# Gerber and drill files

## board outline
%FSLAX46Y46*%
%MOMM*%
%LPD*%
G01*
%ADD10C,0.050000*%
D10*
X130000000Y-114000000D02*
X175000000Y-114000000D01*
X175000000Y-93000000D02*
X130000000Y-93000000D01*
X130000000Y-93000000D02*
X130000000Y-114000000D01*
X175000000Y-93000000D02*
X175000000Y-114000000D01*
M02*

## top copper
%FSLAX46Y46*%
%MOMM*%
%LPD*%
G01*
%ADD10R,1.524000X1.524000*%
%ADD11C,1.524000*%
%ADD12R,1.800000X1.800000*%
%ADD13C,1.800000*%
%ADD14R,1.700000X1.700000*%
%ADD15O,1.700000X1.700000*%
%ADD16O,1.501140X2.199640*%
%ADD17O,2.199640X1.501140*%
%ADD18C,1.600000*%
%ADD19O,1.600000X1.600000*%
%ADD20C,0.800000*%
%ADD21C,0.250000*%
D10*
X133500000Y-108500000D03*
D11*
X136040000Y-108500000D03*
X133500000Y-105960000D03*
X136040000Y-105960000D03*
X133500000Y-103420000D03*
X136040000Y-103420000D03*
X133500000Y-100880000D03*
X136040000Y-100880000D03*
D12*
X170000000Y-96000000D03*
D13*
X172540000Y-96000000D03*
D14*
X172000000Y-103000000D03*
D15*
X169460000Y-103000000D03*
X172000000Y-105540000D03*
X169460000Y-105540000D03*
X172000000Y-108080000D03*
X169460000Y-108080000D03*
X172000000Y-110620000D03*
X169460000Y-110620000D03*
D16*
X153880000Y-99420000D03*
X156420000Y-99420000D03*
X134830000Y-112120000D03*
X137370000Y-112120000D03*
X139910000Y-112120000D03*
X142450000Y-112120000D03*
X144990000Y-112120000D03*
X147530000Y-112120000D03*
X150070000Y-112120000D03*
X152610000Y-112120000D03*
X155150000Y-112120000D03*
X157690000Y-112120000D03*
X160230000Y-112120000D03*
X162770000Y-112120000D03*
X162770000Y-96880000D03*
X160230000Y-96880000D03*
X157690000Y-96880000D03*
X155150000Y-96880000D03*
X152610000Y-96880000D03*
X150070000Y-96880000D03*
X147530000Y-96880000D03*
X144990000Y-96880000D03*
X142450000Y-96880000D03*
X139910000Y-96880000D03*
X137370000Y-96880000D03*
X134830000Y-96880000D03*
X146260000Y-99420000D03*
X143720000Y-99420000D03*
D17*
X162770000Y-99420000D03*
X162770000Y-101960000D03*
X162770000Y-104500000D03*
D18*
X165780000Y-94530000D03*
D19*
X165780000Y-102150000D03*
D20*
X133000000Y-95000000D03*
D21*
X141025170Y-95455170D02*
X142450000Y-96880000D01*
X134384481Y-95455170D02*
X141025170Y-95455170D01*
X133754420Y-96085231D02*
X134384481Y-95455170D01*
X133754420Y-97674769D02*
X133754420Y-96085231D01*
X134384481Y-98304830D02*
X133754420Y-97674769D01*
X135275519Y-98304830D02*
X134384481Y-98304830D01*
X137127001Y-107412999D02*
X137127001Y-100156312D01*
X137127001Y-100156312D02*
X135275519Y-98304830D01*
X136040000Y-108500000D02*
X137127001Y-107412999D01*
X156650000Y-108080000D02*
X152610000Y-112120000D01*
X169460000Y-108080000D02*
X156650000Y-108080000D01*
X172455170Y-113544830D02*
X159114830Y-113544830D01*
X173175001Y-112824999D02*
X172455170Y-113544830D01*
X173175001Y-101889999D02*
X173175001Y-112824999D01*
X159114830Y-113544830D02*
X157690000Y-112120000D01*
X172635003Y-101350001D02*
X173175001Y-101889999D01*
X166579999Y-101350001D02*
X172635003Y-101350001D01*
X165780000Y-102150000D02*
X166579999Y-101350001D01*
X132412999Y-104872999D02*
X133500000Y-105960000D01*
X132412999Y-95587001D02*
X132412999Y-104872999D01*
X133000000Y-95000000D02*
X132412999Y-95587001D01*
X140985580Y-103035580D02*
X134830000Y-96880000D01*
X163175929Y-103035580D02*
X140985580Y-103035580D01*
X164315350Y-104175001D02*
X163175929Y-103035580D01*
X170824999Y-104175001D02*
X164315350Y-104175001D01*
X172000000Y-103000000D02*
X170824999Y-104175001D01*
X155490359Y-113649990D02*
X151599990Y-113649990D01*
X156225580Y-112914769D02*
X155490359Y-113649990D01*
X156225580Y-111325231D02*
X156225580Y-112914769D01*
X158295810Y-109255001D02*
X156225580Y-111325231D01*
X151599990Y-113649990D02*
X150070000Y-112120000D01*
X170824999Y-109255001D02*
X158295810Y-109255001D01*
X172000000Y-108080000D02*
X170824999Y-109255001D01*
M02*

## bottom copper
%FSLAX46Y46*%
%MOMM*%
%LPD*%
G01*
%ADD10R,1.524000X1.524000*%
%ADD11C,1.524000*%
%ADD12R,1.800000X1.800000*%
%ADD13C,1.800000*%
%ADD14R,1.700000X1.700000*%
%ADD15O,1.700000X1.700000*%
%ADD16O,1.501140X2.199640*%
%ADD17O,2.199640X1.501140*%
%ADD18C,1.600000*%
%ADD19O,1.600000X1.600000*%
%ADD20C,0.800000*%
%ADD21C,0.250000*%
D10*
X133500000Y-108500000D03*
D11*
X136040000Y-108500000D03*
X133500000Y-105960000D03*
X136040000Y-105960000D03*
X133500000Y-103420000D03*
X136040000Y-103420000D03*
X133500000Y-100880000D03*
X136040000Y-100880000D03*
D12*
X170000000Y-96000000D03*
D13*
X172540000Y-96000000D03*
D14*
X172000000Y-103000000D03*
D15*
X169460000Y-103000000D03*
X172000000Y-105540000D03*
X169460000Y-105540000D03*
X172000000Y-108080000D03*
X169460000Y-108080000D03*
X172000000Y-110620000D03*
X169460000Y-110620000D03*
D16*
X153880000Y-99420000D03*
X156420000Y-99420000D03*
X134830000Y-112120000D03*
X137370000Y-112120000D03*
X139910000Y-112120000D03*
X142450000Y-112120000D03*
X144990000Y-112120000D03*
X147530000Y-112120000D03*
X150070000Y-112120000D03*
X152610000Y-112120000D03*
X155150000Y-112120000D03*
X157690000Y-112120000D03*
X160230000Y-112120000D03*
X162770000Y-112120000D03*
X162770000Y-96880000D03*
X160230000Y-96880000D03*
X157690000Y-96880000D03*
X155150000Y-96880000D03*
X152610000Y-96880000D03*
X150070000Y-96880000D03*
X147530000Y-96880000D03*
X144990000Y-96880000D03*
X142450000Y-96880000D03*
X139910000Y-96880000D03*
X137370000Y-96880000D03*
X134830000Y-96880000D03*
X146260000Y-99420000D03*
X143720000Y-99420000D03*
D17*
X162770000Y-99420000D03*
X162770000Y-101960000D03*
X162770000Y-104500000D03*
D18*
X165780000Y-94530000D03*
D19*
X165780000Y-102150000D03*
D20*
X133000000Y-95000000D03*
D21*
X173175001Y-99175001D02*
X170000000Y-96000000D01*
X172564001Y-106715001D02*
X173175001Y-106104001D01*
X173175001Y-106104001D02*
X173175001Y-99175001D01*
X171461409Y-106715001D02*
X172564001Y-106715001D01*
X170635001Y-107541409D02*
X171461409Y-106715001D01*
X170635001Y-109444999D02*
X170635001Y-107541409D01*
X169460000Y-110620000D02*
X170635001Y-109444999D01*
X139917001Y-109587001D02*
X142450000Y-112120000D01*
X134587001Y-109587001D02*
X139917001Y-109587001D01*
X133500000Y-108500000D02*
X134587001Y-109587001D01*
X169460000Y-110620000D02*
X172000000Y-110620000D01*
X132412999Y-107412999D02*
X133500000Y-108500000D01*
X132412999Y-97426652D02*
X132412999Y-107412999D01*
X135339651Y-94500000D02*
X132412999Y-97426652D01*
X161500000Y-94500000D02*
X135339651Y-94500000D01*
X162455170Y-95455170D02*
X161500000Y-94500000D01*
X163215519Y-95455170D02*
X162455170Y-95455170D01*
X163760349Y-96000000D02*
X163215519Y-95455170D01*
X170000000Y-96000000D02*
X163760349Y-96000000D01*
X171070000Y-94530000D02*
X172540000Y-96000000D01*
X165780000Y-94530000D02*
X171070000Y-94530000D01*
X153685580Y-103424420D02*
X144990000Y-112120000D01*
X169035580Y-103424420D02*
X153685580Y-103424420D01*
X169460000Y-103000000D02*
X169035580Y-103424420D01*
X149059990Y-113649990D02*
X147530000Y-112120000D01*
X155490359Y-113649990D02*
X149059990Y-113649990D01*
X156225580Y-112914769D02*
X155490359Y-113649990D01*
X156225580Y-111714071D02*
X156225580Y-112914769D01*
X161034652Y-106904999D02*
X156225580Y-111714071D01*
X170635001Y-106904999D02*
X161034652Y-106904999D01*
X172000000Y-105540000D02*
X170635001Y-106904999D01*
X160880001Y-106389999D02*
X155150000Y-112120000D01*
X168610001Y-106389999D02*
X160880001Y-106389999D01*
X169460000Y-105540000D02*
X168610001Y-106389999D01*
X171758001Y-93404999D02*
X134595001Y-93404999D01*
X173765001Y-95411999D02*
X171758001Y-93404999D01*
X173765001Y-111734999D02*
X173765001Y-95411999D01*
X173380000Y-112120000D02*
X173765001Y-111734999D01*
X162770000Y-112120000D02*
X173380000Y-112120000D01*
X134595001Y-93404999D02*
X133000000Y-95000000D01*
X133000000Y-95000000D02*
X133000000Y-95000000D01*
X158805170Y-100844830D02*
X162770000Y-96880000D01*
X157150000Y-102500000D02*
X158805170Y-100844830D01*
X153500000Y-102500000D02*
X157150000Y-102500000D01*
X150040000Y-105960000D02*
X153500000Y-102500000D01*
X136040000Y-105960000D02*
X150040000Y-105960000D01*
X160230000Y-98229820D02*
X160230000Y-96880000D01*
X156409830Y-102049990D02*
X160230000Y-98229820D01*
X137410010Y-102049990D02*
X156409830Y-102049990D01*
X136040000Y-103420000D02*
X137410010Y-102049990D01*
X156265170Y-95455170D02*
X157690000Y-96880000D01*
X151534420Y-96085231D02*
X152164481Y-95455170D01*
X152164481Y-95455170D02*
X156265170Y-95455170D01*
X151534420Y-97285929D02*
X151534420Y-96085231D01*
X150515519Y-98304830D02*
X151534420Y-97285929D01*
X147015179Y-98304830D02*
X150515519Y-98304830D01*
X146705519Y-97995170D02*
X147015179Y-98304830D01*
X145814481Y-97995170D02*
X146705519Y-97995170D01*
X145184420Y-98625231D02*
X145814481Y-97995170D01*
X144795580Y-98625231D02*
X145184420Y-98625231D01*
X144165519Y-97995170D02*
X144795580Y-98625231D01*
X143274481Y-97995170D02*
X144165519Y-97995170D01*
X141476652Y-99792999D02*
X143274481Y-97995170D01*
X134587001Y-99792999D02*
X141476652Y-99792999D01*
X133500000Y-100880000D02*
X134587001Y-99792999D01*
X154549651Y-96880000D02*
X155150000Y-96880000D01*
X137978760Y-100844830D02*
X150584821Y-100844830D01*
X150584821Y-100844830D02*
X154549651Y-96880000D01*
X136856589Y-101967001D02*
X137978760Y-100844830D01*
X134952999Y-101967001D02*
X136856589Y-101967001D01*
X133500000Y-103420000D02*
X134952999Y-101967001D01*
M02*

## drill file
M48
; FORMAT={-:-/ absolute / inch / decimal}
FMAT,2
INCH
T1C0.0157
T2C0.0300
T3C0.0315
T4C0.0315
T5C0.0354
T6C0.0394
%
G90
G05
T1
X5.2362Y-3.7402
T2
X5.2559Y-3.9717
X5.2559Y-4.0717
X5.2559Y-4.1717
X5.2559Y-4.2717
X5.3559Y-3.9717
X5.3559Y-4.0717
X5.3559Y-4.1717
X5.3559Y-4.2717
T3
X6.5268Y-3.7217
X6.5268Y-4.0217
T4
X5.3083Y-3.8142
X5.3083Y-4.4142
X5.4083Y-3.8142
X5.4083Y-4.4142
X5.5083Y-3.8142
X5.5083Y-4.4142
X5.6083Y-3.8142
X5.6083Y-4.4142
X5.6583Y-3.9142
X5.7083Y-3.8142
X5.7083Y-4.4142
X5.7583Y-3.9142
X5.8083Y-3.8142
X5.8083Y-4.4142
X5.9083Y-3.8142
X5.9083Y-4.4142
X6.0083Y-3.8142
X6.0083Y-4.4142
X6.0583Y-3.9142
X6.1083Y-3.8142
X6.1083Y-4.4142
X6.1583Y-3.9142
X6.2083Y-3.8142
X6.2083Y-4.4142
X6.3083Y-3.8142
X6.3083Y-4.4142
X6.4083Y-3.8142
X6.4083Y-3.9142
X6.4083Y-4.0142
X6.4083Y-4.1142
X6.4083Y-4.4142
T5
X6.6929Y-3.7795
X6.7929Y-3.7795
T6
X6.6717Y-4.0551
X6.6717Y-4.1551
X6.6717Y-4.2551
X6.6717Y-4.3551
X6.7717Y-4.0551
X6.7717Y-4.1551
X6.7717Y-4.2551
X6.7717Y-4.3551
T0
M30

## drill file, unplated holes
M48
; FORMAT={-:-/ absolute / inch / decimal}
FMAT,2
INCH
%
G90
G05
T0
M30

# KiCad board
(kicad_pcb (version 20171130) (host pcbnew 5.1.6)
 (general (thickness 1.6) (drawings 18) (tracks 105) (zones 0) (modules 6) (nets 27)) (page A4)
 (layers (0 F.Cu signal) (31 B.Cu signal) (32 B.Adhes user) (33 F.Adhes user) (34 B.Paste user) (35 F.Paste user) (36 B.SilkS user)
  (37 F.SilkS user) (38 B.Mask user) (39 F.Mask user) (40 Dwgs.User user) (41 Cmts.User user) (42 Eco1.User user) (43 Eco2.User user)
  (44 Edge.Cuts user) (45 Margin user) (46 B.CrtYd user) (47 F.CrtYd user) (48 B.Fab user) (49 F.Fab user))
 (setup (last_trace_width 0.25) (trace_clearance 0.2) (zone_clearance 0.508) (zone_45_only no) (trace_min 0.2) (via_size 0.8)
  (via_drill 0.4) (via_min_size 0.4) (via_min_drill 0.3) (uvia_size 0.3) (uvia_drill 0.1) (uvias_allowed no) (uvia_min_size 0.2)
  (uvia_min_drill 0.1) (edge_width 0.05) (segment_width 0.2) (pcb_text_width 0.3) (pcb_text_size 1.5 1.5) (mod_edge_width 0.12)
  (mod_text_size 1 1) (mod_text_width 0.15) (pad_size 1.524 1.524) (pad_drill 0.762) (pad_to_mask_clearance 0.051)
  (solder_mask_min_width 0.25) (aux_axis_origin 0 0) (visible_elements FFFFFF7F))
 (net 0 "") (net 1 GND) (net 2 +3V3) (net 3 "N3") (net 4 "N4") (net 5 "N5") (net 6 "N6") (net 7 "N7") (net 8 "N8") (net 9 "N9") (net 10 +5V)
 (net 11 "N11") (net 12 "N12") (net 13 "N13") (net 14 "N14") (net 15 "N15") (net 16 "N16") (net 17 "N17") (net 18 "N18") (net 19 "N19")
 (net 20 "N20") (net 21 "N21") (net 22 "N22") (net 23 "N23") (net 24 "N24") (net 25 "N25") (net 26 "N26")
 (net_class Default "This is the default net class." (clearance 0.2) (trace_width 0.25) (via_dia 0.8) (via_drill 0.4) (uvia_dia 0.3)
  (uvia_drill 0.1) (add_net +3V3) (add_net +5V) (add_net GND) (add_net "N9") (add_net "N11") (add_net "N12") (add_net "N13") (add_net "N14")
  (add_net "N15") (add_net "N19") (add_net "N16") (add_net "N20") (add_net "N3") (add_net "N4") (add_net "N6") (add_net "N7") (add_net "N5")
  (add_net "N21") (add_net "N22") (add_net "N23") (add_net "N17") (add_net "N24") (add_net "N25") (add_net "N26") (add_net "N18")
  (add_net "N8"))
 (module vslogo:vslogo (layer B.Cu) (at 150 105.5 180)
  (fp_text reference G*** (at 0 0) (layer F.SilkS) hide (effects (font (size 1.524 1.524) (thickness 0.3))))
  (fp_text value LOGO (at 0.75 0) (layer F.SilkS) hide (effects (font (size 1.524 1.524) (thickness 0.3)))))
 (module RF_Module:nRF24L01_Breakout (layer B.Cu) (at 133.5 108.5)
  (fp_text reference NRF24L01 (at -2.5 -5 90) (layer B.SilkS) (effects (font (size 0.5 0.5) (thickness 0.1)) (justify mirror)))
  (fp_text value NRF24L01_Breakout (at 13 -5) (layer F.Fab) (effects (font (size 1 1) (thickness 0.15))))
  (pad 1 thru_hole rect (at 0 0) (size 1.524 1.524) (drill 0.762) (layers *.Cu *.Mask) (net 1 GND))
  (pad 2 thru_hole circle (at 2.54 0) (size 1.524 1.524) (drill 0.762) (layers *.Cu *.Mask) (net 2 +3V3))
  (pad 3 thru_hole circle (at 0 -2.54) (size 1.524 1.524) (drill 0.762) (layers *.Cu *.Mask) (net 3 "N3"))
  (pad 4 thru_hole circle (at 2.54 -2.54) (size 1.524 1.524) (drill 0.762) (layers *.Cu *.Mask) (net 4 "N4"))
  (pad 5 thru_hole circle (at 0 -5.08) (size 1.524 1.524) (drill 0.762) (layers *.Cu *.Mask) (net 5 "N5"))
  (pad 6 thru_hole circle (at 2.54 -5.08) (size 1.524 1.524) (drill 0.762) (layers *.Cu *.Mask) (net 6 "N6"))
  (pad 7 thru_hole circle (at 0 -7.62) (size 1.524 1.524) (drill 0.762) (layers *.Cu *.Mask) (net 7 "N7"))
  (pad 8 thru_hole circle (at 2.54 -7.62) (size 1.524 1.524) (drill 0.762) (layers *.Cu *.Mask) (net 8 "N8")))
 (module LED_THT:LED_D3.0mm (layer F.Cu) (at 170 96)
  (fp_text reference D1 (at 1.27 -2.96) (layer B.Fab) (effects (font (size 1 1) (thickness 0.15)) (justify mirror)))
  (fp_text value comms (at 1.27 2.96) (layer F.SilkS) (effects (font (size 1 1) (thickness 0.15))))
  (pad 1 thru_hole rect (at 0 0) (size 1.8 1.8) (drill 0.9) (layers *.Cu *.Mask) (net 1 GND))
  (pad 2 thru_hole circle (at 2.54 0) (size 1.8 1.8) (drill 0.9) (layers *.Cu *.Mask) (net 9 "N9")))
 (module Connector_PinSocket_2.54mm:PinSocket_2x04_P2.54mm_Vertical (layer F.Cu) (at 172 103)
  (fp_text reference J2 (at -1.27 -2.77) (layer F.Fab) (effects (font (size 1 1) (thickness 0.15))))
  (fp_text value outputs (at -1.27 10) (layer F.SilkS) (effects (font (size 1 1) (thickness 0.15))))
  (pad 1 thru_hole rect (at 0 0) (size 1.7 1.7) (drill 1) (layers *.Cu *.Mask) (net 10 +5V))
  (pad 2 thru_hole oval (at -2.54 0) (size 1.7 1.7) (drill 1) (layers *.Cu *.Mask) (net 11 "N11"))
  (pad 3 thru_hole oval (at 0 2.54) (size 1.7 1.7) (drill 1) (layers *.Cu *.Mask) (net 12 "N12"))
  (pad 4 thru_hole oval (at -2.54 2.54) (size 1.7 1.7) (drill 1) (layers *.Cu *.Mask) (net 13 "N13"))
  (pad 5 thru_hole oval (at 0 5.08) (size 1.7 1.7) (drill 1) (layers *.Cu *.Mask) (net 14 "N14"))
  (pad 6 thru_hole oval (at -2.54 5.08) (size 1.7 1.7) (drill 1) (layers *.Cu *.Mask) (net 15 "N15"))
  (pad 7 thru_hole oval (at 0 7.62) (size 1.7 1.7) (drill 1) (layers *.Cu *.Mask) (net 1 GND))
  (pad 8 thru_hole oval (at -2.54 7.62) (size 1.7 1.7) (drill 1) (layers *.Cu *.Mask) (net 1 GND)))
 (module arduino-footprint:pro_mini (layer F.Cu) (at 148.8 104.5)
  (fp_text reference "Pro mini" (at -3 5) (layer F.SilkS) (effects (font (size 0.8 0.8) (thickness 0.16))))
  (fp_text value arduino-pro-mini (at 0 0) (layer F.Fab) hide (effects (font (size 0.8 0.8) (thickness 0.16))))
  (pad 28 thru_hole oval (at 5.08 -5.08) (size 1.50114 2.19964) (drill 0.8001) (layers *.Cu *.Mask F.SilkS))
  (pad 27 thru_hole oval (at 7.62 -5.08) (size 1.50114 2.19964) (drill 0.8001) (layers *.Cu *.Mask F.SilkS))
  (pad 1 thru_hole oval (at -13.97 7.62) (size 1.50114 2.19964) (drill 0.8001) (layers *.Cu *.Mask F.SilkS) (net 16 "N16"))
  (pad 2 thru_hole oval (at -11.43 7.62) (size 1.50114 2.19964) (drill 0.8001) (layers *.Cu *.Mask F.SilkS) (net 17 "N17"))
  (pad 3 thru_hole oval (at -8.89 7.62) (size 1.50114 2.19964) (drill 0.8001) (layers *.Cu *.Mask F.SilkS) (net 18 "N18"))
  (pad 4 thru_hole oval (at -6.35 7.62) (size 1.50114 2.19964) (drill 0.8001) (layers *.Cu *.Mask F.SilkS) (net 1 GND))
  (pad 5 thru_hole oval (at -3.81 7.62) (size 1.50114 2.19964) (drill 0.8001) (layers *.Cu *.Mask F.SilkS) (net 11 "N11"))
  (pad 6 thru_hole oval (at -1.27 7.62) (size 1.50114 2.19964) (drill 0.8001) (layers *.Cu *.Mask F.SilkS) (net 12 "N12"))
  (pad 7 thru_hole oval (at 1.27 7.62) (size 1.50114 2.19964) (drill 0.8001) (layers *.Cu *.Mask F.SilkS) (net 14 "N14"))
  (pad 8 thru_hole oval (at 3.81 7.62) (size 1.50114 2.19964) (drill 0.8001) (layers *.Cu *.Mask F.SilkS) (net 15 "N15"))
  (pad 9 thru_hole oval (at 6.35 7.62) (size 1.50114 2.19964) (drill 0.8001) (layers *.Cu *.Mask F.SilkS) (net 13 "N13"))
  (pad 10 thru_hole oval (at 8.89 7.62) (size 1.50114 2.19964) (drill 0.8001) (layers *.Cu *.Mask F.SilkS) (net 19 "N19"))
  (pad 11 thru_hole oval (at 11.43 7.62) (size 1.50114 2.19964) (drill 0.8001) (layers *.Cu *.Mask F.SilkS) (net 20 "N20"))
  (pad 12 thru_hole oval (at 13.97 7.62) (size 1.50114 2.19964) (drill 0.8001) (layers *.Cu *.Mask F.SilkS) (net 3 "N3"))
  (pad 13 thru_hole oval (at 13.97 -7.62) (size 1.50114 2.19964) (drill 0.8001) (layers *.Cu *.Mask F.SilkS) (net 4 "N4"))
  (pad 14 thru_hole oval (at 11.43 -7.62) (size 1.50114 2.19964) (drill 0.8001) (layers *.Cu *.Mask F.SilkS) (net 6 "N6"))
  (pad 15 thru_hole oval (at 8.89 -7.62) (size 1.50114 2.19964) (drill 0.8001) (layers *.Cu *.Mask F.SilkS) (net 7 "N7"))
  (pad 16 thru_hole oval (at 6.35 -7.62) (size 1.50114 2.19964) (drill 0.8001) (layers *.Cu *.Mask F.SilkS) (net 5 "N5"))
  (pad 17 thru_hole oval (at 3.81 -7.62) (size 1.50114 2.19964) (drill 0.8001) (layers *.Cu *.Mask F.SilkS) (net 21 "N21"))
  (pad 18 thru_hole oval (at 1.27 -7.62) (size 1.50114 2.19964) (drill 0.8001) (layers *.Cu *.Mask F.SilkS) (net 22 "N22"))
  (pad 19 thru_hole oval (at -1.27 -7.62) (size 1.50114 2.19964) (drill 0.8001) (layers *.Cu *.Mask F.SilkS) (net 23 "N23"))
  (pad 20 thru_hole oval (at -3.81 -7.62) (size 1.50114 2.19964) (drill 0.8001) (layers *.Cu *.Mask F.SilkS) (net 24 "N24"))
  (pad 21 thru_hole oval (at -6.35 -7.62) (size 1.50114 2.19964) (drill 0.8001) (layers *.Cu *.Mask F.SilkS) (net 2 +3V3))
  (pad 22 thru_hole oval (at -8.89 -7.62) (size 1.50114 2.19964) (drill 0.8001) (layers *.Cu *.Mask F.SilkS) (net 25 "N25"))
  (pad 23 thru_hole oval (at -11.43 -7.62) (size 1.50114 2.19964) (drill 0.8001) (layers *.Cu *.Mask F.SilkS) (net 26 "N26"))
  (pad 24 thru_hole oval (at -13.97 -7.62) (size 1.50114 2.19964) (drill 0.8001) (layers *.Cu *.Mask F.SilkS) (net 10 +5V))
  (pad 25 thru_hole oval (at -2.54 -5.08) (size 1.50114 2.19964) (drill 0.8001) (layers *.Cu *.Mask F.SilkS))
  (pad 26 thru_hole oval (at -5.08 -5.08) (size 1.50114 2.19964) (drill 0.8001) (layers *.Cu *.Mask F.SilkS))
  (pad 27 thru_hole oval (at 13.97 -5.08) (size 2.19964 1.50114) (drill 0.8001) (layers *.Cu *.Mask F.SilkS))
  (pad 28 thru_hole oval (at 13.97 -2.54) (size 2.19964 1.50114) (drill 0.8001) (layers *.Cu *.Mask F.SilkS))
  (pad 29 thru_hole oval (at 13.97 0) (size 2.19964 1.50114) (drill 0.8001) (layers *.Cu *.Mask F.SilkS)))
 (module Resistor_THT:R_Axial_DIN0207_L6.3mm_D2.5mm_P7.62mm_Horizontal (layer F.Cu) (at 165.78 94.53 270)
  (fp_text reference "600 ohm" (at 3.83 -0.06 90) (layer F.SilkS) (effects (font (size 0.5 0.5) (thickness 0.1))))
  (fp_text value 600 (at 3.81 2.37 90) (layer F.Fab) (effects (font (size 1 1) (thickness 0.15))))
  (pad 1 thru_hole circle (at 0 0 270) (size 1.6 1.6) (drill 0.8) (layers *.Cu *.Mask) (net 9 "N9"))
  (pad 2 thru_hole oval (at 7.62 0 270) (size 1.6 1.6) (drill 0.8) (layers *.Cu *.Mask) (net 19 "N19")))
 (gr_line (start 130 114) (end 175 114) (layer Edge.Cuts) (width 0.05))
 (gr_line (start 175 93) (end 130 93) (layer Edge.Cuts) (width 0.05))
 (gr_line (start 130 93) (end 130 114) (layer Edge.Cuts) (width 0.05))
 (gr_line (start 175 93) (end 175 114) (layer Edge.Cuts) (width 0.05))
 (segment (start 173.175001 99.175001) (end 170 96) (width 0.25) (layer B.Cu) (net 1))
 (segment (start 172.564001 106.715001) (end 173.175001 106.104001) (width 0.25) (layer B.Cu) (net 1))
 (segment (start 173.175001 106.104001) (end 173.175001 99.175001) (width 0.25) (layer B.Cu) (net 1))
 (segment (start 171.461409 106.715001) (end 172.564001 106.715001) (width 0.25) (layer B.Cu) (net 1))
 (segment (start 170.635001 107.541409) (end 171.461409 106.715001) (width 0.25) (layer B.Cu) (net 1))
 (segment (start 170.635001 109.444999) (end 170.635001 107.541409) (width 0.25) (layer B.Cu) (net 1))
 (segment (start 169.46 110.62) (end 170.635001 109.444999) (width 0.25) (layer B.Cu) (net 1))
 (segment (start 139.917001 109.587001) (end 142.45 112.12) (width 0.25) (layer B.Cu) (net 1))
 (segment (start 134.587001 109.587001) (end 139.917001 109.587001) (width 0.25) (layer B.Cu) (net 1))
 (segment (start 133.5 108.5) (end 134.587001 109.587001) (width 0.25) (layer B.Cu) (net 1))
 (segment (start 169.46 110.62) (end 172 110.62) (width 0.25) (layer B.Cu) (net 1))
 (segment (start 132.412999 107.412999) (end 133.5 108.5) (width 0.25) (layer B.Cu) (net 1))
 (segment (start 132.412999 97.426652) (end 132.412999 107.412999) (width 0.25) (layer B.Cu) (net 1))
 (segment (start 135.339651 94.5) (end 132.412999 97.426652) (width 0.25) (layer B.Cu) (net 1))
 (segment (start 161.5 94.5) (end 135.339651 94.5) (width 0.25) (layer B.Cu) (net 1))
 (segment (start 162.45517 95.45517) (end 161.5 94.5) (width 0.25) (layer B.Cu) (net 1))
 (segment (start 163.215519 95.45517) (end 162.45517 95.45517) (width 0.25) (layer B.Cu) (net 1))
 (segment (start 163.760349 96) (end 163.215519 95.45517) (width 0.25) (layer B.Cu) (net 1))
 (segment (start 170 96) (end 163.760349 96) (width 0.25) (layer B.Cu) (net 1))
 (segment (start 171.07 94.53) (end 172.54 96) (width 0.25) (layer B.Cu) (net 9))
 (segment (start 165.78 94.53) (end 171.07 94.53) (width 0.25) (layer B.Cu) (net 9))
 (segment (start 141.02517 95.45517) (end 142.45 96.88) (width 0.25) (layer F.Cu) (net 2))
 (segment (start 134.384481 95.45517) (end 141.02517 95.45517) (width 0.25) (layer F.Cu) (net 2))
 (segment (start 133.75442 96.085231) (end 134.384481 95.45517) (width 0.25) (layer F.Cu) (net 2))
 (segment (start 133.75442 97.674769) (end 133.75442 96.085231) (width 0.25) (layer F.Cu) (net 2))
 (segment (start 134.384481 98.30483) (end 133.75442 97.674769) (width 0.25) (layer F.Cu) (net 2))
 (segment (start 135.275519 98.30483) (end 134.384481 98.30483) (width 0.25) (layer F.Cu) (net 2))
 (segment (start 137.127001 107.412999) (end 137.127001 100.156312) (width 0.25) (layer F.Cu) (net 2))
 (segment (start 137.127001 100.156312) (end 135.275519 98.30483) (width 0.25) (layer F.Cu) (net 2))
 (segment (start 136.04 108.5) (end 137.127001 107.412999) (width 0.25) (layer F.Cu) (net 2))
 (segment (start 153.68558 103.42442) (end 144.99 112.12) (width 0.25) (layer B.Cu) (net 11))
 (segment (start 169.03558 103.42442) (end 153.68558 103.42442) (width 0.25) (layer B.Cu) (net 11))
 (segment (start 169.46 103) (end 169.03558 103.42442) (width 0.25) (layer B.Cu) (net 11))
 (segment (start 149.05999 113.64999) (end 147.53 112.12) (width 0.25) (layer B.Cu) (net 12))
 (segment (start 155.490359 113.64999) (end 149.05999 113.64999) (width 0.25) (layer B.Cu) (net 12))
 (segment (start 156.22558 112.914769) (end 155.490359 113.64999) (width 0.25) (layer B.Cu) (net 12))
 (segment (start 156.22558 111.714071) (end 156.22558 112.914769) (width 0.25) (layer B.Cu) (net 12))
 (segment (start 161.034652 106.904999) (end 156.22558 111.714071) (width 0.25) (layer B.Cu) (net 12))
 (segment (start 170.635001 106.904999) (end 161.034652 106.904999) (width 0.25) (layer B.Cu) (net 12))
 (segment (start 172 105.54) (end 170.635001 106.904999) (width 0.25) (layer B.Cu) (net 12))
 (segment (start 160.880001 106.389999) (end 155.15 112.12) (width 0.25) (layer B.Cu) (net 13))
 (segment (start 168.610001 106.389999) (end 160.880001 106.389999) (width 0.25) (layer B.Cu) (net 13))
 (segment (start 169.46 105.54) (end 168.610001 106.389999) (width 0.25) (layer B.Cu) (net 13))
 (segment (start 156.65 108.08) (end 152.61 112.12) (width 0.25) (layer F.Cu) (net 15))
 (segment (start 169.46 108.08) (end 156.65 108.08) (width 0.25) (layer F.Cu) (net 15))
 (segment (start 172.45517 113.54483) (end 159.11483 113.54483) (width 0.25) (layer F.Cu) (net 19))
 (segment (start 173.175001 112.824999) (end 172.45517 113.54483) (width 0.25) (layer F.Cu) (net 19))
 (segment (start 173.175001 101.889999) (end 173.175001 112.824999) (width 0.25) (layer F.Cu) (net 19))
 (segment (start 159.11483 113.54483) (end 157.69 112.12) (width 0.25) (layer F.Cu) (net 19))
 (segment (start 172.635003 101.350001) (end 173.175001 101.889999) (width 0.25) (layer F.Cu) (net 19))
 (segment (start 166.579999 101.350001) (end 172.635003 101.350001) (width 0.25) (layer F.Cu) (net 19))
 (segment (start 165.78 102.15) (end 166.579999 101.350001) (width 0.25) (layer F.Cu) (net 19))
 (segment (start 171.758001 93.404999) (end 134.595001 93.404999) (width 0.25) (layer B.Cu) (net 3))
 (segment (start 173.765001 95.411999) (end 171.758001 93.404999) (width 0.25) (layer B.Cu) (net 3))
 (segment (start 173.765001 111.734999) (end 173.765001 95.411999) (width 0.25) (layer B.Cu) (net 3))
 (segment (start 173.38 112.12) (end 173.765001 111.734999) (width 0.25) (layer B.Cu) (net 3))
 (segment (start 162.77 112.12) (end 173.38 112.12) (width 0.25) (layer B.Cu) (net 3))
 (segment (start 134.595001 93.404999) (end 133 95) (width 0.25) (layer B.Cu) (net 3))
 (segment (start 133 95) (end 133 95) (width 0.25) (layer B.Cu) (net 3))
 (via (at 133 95) (size 0.8) (drill 0.4) (layers F.Cu B.Cu) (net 3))
 (segment (start 132.412999 104.872999) (end 133.5 105.96) (width 0.25) (layer F.Cu) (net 3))
 (segment (start 132.412999 95.587001) (end 132.412999 104.872999) (width 0.25) (layer F.Cu) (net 3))
 (segment (start 133 95) (end 132.412999 95.587001) (width 0.25) (layer F.Cu) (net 3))
 (segment (start 158.80517 100.84483) (end 162.77 96.88) (width 0.25) (layer B.Cu) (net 4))
 (segment (start 157.15 102.5) (end 158.80517 100.84483) (width 0.25) (layer B.Cu) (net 4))
 (segment (start 153.5 102.5) (end 157.15 102.5) (width 0.25) (layer B.Cu) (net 4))
 (segment (start 150.04 105.96) (end 153.5 102.5) (width 0.25) (layer B.Cu) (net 4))
 (segment (start 136.04 105.96) (end 150.04 105.96) (width 0.25) (layer B.Cu) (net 4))
 (segment (start 160.23 98.22982) (end 160.23 96.88) (width 0.25) (layer B.Cu) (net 6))
 (segment (start 156.40983 102.04999) (end 160.23 98.22982) (width 0.25) (layer B.Cu) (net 6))
 (segment (start 137.41001 102.04999) (end 156.40983 102.04999) (width 0.25) (layer B.Cu) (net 6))
 (segment (start 136.04 103.42) (end 137.41001 102.04999) (width 0.25) (layer B.Cu) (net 6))
 (segment (start 156.26517 95.45517) (end 157.69 96.88) (width 0.25) (layer B.Cu) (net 7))
 (segment (start 151.53442 96.085231) (end 152.164481 95.45517) (width 0.25) (layer B.Cu) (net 7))
 (segment (start 152.164481 95.45517) (end 156.26517 95.45517) (width 0.25) (layer B.Cu) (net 7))
 (segment (start 151.53442 97.285929) (end 151.53442 96.085231) (width 0.25) (layer B.Cu) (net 7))
 (segment (start 150.515519 98.30483) (end 151.53442 97.285929) (width 0.25) (layer B.Cu) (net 7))
 (segment (start 147.015179 98.30483) (end 150.515519 98.30483) (width 0.25) (layer B.Cu) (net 7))
 (segment (start 146.705519 97.99517) (end 147.015179 98.30483) (width 0.25) (layer B.Cu) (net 7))
 (segment (start 145.814481 97.99517) (end 146.705519 97.99517) (width 0.25) (layer B.Cu) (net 7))
 (segment (start 145.18442 98.625231) (end 145.814481 97.99517) (width 0.25) (layer B.Cu) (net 7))
 (segment (start 144.79558 98.625231) (end 145.18442 98.625231) (width 0.25) (layer B.Cu) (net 7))
 (segment (start 144.165519 97.99517) (end 144.79558 98.625231) (width 0.25) (layer B.Cu) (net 7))
 (segment (start 143.274481 97.99517) (end 144.165519 97.99517) (width 0.25) (layer B.Cu) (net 7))
 (segment (start 141.476652 99.792999) (end 143.274481 97.99517) (width 0.25) (layer B.Cu) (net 7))
 (segment (start 134.587001 99.792999) (end 141.476652 99.792999) (width 0.25) (layer B.Cu) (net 7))
 (segment (start 133.5 100.88) (end 134.587001 99.792999) (width 0.25) (layer B.Cu) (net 7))
 (segment (start 154.549651 96.88) (end 155.15 96.88) (width 0.25) (layer B.Cu) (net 5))
 (segment (start 137.97876 100.84483) (end 150.584821 100.84483) (width 0.25) (layer B.Cu) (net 5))
 (segment (start 150.584821 100.84483) (end 154.549651 96.88) (width 0.25) (layer B.Cu) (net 5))
 (segment (start 136.856589 101.967001) (end 137.97876 100.84483) (width 0.25) (layer B.Cu) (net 5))
 (segment (start 134.952999 101.967001) (end 136.856589 101.967001) (width 0.25) (layer B.Cu) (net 5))
 (segment (start 133.5 103.42) (end 134.952999 101.967001) (width 0.25) (layer B.Cu) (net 5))
 (segment (start 140.98558 103.03558) (end 134.83 96.88) (width 0.25) (layer F.Cu) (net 10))
 (segment (start 163.175929 103.03558) (end 140.98558 103.03558) (width 0.25) (layer F.Cu) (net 10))
 (segment (start 164.31535 104.175001) (end 163.175929 103.03558) (width 0.25) (layer F.Cu) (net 10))
 (segment (start 170.824999 104.175001) (end 164.31535 104.175001) (width 0.25) (layer F.Cu) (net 10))
 (segment (start 172 103) (end 170.824999 104.175001) (width 0.25) (layer F.Cu) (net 10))
 (segment (start 155.490359 113.64999) (end 151.59999 113.64999) (width 0.25) (layer F.Cu) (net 14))
 (segment (start 156.22558 112.914769) (end 155.490359 113.64999) (width 0.25) (layer F.Cu) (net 14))
 (segment (start 156.22558 111.325231) (end 156.22558 112.914769) (width 0.25) (layer F.Cu) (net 14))
 (segment (start 158.29581 109.255001) (end 156.22558 111.325231) (width 0.25) (layer F.Cu) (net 14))
 (segment (start 151.59999 113.64999) (end 150.07 112.12) (width 0.25) (layer F.Cu) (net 14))
 (segment (start 170.824999 109.255001) (end 158.29581 109.255001) (width 0.25) (layer F.Cu) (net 14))
 (segment (start 172 108.08) (end 170.824999 109.255001) (width 0.25) (layer F.Cu) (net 14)))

